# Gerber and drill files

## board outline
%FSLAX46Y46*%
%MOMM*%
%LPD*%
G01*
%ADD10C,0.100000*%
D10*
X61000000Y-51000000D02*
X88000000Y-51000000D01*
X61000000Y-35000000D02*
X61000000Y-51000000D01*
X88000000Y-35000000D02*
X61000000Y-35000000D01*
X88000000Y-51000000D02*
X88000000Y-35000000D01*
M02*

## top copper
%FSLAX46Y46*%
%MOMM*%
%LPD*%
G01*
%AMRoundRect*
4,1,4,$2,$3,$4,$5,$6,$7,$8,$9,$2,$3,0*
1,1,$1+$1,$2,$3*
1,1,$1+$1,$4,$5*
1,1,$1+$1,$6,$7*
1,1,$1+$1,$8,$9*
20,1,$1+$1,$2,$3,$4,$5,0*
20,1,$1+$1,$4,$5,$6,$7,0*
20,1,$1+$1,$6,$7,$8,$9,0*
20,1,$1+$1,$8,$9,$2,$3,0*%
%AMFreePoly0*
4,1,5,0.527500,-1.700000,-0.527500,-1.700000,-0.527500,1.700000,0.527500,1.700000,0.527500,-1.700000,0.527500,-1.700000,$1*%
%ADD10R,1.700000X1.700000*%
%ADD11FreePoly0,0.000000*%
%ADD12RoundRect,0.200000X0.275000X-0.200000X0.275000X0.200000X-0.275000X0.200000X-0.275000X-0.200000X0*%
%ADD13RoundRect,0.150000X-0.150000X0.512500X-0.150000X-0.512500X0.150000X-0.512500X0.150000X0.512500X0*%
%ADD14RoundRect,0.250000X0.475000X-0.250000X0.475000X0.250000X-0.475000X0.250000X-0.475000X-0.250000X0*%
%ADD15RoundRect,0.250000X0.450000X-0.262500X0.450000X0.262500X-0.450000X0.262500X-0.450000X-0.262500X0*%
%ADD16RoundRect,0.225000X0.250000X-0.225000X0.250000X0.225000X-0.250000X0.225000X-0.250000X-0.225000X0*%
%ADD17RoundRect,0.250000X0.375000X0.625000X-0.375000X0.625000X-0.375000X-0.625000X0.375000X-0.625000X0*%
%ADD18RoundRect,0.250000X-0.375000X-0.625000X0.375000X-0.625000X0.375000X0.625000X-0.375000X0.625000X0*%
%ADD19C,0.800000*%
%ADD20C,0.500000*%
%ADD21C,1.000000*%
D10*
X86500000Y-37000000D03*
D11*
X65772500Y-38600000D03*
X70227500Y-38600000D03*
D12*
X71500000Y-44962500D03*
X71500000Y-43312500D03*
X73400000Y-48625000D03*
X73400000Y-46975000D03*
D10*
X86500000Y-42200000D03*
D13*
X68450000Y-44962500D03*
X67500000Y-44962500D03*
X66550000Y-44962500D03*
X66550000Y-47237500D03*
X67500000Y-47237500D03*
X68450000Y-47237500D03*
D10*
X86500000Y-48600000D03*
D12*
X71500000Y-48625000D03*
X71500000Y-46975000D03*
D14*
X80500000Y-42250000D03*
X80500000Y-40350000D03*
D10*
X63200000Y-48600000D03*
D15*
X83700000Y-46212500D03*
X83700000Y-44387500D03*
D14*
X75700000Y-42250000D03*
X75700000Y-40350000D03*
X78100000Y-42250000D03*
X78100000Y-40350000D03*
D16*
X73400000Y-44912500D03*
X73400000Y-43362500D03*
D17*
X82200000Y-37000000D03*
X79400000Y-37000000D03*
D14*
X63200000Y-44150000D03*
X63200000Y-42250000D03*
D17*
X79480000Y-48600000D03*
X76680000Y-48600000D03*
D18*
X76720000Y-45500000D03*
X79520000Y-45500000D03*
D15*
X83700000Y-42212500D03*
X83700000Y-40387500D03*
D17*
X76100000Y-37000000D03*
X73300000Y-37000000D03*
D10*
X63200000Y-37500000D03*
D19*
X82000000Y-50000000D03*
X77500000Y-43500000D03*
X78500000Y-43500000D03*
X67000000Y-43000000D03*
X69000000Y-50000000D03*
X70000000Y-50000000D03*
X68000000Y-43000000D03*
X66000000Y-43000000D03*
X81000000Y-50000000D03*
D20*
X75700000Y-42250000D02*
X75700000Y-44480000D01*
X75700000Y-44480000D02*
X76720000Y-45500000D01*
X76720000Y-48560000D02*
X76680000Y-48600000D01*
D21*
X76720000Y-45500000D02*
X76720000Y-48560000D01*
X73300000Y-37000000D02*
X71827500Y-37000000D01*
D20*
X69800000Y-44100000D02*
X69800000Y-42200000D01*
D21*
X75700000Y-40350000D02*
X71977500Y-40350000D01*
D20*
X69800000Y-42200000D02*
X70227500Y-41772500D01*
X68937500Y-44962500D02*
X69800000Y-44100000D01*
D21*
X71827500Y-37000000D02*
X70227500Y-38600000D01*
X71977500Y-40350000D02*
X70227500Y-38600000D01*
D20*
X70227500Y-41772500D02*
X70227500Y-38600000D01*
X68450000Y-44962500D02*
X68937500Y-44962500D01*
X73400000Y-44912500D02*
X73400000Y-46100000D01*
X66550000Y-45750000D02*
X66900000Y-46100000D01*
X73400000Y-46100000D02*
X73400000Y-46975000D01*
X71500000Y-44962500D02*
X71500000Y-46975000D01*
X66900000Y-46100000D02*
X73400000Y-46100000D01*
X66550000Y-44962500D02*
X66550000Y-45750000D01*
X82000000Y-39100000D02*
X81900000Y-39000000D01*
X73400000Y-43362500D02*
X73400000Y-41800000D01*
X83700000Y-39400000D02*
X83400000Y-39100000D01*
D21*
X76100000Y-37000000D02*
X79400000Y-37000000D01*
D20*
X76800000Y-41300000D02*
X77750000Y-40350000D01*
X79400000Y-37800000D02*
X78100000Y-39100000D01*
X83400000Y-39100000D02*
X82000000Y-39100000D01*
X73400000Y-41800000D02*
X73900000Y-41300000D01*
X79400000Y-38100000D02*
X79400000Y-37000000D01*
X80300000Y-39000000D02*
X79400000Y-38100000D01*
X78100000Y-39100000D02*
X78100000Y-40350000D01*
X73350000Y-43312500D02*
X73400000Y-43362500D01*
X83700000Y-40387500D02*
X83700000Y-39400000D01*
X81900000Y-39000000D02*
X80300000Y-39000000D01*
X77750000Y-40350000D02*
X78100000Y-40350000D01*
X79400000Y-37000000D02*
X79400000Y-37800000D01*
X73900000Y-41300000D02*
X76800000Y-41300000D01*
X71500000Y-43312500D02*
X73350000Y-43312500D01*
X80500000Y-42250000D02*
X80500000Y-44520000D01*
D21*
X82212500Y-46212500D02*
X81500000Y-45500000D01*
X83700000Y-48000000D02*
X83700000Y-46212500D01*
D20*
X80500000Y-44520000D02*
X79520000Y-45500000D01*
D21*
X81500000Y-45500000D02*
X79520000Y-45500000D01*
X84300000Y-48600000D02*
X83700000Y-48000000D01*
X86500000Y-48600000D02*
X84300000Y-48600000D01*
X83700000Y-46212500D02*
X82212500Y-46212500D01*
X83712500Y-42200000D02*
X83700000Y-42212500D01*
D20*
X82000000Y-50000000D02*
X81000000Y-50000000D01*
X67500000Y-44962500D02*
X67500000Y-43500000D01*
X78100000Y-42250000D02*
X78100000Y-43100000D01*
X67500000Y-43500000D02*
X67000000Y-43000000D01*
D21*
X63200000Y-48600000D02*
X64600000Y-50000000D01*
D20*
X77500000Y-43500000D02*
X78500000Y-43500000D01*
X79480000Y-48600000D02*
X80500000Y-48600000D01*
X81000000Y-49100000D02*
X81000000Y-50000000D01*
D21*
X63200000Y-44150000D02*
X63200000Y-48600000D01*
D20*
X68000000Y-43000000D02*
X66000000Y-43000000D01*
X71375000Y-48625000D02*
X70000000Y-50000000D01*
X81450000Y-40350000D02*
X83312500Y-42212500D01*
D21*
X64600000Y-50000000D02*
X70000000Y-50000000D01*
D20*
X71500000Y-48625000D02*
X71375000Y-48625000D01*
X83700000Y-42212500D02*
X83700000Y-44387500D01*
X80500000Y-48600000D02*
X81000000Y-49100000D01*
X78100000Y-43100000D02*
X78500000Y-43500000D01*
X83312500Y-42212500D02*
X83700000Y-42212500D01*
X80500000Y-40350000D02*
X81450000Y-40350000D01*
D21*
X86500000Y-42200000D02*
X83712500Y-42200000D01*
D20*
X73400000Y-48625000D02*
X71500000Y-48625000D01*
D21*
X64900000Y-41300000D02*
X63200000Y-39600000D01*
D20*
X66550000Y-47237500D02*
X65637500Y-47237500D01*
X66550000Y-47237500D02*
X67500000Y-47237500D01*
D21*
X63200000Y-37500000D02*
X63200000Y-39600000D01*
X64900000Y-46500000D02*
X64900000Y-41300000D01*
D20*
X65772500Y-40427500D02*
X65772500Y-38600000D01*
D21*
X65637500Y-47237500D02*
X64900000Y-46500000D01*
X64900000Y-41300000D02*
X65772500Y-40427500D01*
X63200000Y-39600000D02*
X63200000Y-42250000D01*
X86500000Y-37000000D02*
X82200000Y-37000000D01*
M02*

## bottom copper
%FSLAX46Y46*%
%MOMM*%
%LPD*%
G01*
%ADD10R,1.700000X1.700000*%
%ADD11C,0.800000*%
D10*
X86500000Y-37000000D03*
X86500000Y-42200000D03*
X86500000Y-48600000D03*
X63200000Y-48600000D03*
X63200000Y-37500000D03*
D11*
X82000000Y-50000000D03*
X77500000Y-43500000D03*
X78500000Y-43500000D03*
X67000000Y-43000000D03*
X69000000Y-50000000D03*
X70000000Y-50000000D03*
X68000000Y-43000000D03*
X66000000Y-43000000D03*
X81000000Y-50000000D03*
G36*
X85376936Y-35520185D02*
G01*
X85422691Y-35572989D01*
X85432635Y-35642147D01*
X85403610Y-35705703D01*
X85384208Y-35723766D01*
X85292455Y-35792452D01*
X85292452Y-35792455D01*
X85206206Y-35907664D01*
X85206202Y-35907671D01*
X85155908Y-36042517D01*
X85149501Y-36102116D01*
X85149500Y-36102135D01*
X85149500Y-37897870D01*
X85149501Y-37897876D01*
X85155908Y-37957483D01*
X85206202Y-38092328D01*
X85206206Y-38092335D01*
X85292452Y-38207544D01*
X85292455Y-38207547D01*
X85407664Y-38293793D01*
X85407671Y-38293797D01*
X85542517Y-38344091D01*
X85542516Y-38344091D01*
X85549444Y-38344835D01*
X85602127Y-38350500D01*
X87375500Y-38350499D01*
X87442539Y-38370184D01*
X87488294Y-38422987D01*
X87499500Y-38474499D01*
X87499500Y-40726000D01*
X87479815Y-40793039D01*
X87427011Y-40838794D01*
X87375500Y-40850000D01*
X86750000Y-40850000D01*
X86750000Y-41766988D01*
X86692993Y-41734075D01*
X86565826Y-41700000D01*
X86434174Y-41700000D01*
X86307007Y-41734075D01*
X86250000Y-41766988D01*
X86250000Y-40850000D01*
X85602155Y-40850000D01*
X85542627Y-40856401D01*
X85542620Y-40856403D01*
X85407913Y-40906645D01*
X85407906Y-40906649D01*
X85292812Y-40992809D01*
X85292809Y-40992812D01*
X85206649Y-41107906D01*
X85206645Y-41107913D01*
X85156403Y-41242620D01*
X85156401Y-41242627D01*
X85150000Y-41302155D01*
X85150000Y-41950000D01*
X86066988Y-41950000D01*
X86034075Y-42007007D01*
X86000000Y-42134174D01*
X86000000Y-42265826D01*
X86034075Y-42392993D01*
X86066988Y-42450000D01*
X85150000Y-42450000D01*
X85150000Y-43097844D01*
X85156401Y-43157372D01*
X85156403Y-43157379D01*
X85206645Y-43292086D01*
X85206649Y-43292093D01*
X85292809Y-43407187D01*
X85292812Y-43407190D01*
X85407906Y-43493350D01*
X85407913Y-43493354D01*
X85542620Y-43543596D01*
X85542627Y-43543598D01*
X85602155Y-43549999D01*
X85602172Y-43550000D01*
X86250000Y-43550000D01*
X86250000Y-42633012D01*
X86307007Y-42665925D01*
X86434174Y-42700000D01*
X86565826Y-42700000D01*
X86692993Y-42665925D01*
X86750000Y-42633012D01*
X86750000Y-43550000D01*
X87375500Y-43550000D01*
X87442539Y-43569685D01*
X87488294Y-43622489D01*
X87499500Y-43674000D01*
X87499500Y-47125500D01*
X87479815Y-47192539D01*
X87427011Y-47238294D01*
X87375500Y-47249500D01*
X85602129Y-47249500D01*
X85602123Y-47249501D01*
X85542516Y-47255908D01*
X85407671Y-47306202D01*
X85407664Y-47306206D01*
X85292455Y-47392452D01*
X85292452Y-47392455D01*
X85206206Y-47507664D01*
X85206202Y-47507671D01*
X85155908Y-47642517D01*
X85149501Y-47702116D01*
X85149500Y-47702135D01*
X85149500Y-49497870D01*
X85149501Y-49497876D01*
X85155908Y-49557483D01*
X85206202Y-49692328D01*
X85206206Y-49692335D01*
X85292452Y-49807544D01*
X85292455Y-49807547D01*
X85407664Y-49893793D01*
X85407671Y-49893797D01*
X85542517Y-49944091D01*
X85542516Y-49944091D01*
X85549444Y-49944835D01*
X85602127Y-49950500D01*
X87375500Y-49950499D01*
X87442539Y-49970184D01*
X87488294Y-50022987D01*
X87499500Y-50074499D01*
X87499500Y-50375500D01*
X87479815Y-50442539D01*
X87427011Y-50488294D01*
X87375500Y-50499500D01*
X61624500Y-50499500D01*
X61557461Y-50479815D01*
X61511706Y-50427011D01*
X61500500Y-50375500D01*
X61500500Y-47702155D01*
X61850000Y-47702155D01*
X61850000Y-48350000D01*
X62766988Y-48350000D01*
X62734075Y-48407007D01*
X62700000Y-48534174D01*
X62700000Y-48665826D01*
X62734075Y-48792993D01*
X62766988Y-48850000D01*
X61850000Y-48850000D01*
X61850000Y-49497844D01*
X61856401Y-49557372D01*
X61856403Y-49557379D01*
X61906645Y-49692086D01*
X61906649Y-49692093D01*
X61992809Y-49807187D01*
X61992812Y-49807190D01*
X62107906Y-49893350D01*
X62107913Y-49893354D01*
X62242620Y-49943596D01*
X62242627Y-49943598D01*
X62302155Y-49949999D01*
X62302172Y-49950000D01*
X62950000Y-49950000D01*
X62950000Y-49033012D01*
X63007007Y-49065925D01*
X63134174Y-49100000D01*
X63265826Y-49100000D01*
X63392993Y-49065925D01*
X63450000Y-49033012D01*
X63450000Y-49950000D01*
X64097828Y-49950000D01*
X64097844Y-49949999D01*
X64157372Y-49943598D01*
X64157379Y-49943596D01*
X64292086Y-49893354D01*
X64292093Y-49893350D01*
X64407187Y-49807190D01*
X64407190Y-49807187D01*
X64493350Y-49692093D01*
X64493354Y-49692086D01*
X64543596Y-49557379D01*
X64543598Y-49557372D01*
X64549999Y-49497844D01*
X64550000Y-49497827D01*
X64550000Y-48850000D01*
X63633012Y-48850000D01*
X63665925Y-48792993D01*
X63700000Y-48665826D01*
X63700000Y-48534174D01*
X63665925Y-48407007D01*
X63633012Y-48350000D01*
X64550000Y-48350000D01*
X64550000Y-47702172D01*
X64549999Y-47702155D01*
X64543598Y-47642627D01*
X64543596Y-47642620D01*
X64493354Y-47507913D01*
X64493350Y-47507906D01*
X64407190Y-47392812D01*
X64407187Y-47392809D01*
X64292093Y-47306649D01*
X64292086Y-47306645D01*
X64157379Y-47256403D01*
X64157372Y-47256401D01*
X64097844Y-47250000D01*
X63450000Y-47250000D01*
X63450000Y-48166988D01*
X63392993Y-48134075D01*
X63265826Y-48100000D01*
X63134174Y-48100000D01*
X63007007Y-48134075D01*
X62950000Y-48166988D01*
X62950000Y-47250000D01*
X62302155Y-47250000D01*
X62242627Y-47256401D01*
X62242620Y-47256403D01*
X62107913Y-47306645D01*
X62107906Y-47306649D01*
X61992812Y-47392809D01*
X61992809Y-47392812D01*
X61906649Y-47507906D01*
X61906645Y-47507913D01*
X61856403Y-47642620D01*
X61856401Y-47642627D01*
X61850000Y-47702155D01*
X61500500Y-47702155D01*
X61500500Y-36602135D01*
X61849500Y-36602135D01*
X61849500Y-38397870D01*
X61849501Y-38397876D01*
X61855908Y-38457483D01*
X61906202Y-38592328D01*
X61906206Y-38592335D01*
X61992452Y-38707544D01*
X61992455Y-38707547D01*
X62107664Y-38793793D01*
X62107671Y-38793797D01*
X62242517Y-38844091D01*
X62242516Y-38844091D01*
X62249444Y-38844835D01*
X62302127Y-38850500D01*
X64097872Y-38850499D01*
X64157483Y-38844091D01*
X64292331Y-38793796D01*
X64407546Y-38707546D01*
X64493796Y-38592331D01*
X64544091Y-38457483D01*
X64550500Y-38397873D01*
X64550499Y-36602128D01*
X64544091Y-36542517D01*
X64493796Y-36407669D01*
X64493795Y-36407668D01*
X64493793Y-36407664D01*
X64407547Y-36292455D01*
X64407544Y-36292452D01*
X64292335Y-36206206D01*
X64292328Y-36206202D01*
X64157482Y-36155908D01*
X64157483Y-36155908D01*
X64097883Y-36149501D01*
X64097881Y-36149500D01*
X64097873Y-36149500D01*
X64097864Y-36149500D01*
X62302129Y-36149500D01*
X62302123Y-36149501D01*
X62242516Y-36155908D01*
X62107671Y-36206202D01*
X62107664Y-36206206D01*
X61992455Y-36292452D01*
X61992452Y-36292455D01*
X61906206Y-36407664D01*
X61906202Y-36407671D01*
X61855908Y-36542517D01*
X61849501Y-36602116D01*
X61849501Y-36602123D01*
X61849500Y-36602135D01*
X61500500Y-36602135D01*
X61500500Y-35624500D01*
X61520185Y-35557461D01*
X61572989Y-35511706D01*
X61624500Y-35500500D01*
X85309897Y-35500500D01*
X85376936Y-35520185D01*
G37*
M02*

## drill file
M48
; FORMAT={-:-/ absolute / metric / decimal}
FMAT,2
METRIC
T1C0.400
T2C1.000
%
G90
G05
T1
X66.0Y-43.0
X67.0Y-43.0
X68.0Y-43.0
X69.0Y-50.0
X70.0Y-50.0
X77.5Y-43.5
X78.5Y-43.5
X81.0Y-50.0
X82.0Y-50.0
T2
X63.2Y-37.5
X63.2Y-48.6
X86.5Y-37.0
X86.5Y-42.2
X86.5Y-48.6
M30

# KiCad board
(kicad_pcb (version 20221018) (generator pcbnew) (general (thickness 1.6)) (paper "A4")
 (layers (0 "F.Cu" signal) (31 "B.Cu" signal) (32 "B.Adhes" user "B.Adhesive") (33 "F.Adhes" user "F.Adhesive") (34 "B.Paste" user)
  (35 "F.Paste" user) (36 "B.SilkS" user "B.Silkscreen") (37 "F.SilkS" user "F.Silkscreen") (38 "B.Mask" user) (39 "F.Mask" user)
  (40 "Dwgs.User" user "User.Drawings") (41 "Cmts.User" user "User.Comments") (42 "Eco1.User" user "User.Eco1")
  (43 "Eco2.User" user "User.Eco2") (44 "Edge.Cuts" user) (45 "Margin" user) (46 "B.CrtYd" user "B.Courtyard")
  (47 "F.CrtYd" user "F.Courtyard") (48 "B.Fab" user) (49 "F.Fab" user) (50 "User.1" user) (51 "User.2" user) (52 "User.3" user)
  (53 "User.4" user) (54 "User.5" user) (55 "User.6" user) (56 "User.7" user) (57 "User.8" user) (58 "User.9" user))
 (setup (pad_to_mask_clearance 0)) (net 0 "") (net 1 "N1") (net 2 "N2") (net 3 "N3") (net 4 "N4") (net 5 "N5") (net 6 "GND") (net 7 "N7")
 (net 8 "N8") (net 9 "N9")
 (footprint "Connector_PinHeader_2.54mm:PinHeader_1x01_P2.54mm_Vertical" (layer "F.Cu") (at 86.5 37)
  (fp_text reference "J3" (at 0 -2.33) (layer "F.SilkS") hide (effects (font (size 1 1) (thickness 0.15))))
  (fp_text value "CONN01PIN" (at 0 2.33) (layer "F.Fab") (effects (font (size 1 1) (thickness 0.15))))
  (pad "1" thru_hole rect (at 0 0) (size 1.7 1.7) (drill 1) (layers "*.Cu" "*.Mask") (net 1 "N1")))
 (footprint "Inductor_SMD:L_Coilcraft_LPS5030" (layer "F.Cu") (at 68 38.6)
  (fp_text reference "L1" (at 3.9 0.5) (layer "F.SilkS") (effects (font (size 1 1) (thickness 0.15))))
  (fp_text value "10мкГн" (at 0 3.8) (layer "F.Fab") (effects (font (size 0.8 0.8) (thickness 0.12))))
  (pad "1" smd custom (at -2.2275 0) (size 1.055 3.4) (layers "F.Cu" "F.Paste" "F.Mask") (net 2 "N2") (zone_connect 2)
   (options (clearance outline) (anchor rect)) (primitives))
  (pad "2" smd custom (at 2.2275 0) (size 1.055 3.4) (layers "F.Cu" "F.Paste" "F.Mask") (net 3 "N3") (zone_connect 2)
   (options (clearance outline) (anchor rect)) (primitives)))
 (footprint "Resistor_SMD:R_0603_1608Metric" (layer "F.Cu") (at 71.5 44.1375 90)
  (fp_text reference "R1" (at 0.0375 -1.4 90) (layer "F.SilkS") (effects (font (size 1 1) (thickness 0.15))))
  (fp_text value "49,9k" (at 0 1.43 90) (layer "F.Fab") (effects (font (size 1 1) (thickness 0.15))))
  (pad "1" smd roundrect (at -0.825 0 90) (size 0.8 0.95) (layers "F.Cu" "F.Paste" "F.Mask") (roundrect_rratio 0.25) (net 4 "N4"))
  (pad "2" smd roundrect (at 0.825 0 90) (size 0.8 0.95) (layers "F.Cu" "F.Paste" "F.Mask") (roundrect_rratio 0.25) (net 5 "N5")))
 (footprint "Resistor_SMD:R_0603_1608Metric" (layer "F.Cu") (at 73.4 47.8 90)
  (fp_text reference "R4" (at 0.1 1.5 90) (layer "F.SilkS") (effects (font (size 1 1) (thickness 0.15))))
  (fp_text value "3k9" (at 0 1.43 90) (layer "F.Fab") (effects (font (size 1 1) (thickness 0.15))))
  (pad "1" smd roundrect (at -0.825 0 90) (size 0.8 0.95) (layers "F.Cu" "F.Paste" "F.Mask") (roundrect_rratio 0.25) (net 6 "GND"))
  (pad "2" smd roundrect (at 0.825 0 90) (size 0.8 0.95) (layers "F.Cu" "F.Paste" "F.Mask") (roundrect_rratio 0.25) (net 4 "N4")))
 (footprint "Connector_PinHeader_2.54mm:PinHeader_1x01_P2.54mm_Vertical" (layer "F.Cu") (at 86.5 42.2)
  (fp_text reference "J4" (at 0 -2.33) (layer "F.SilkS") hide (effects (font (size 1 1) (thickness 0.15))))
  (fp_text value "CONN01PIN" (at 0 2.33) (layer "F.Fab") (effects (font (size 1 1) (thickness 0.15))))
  (pad "1" thru_hole rect (at 0 0) (size 1.7 1.7) (drill 1) (layers "*.Cu" "*.Mask") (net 6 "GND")))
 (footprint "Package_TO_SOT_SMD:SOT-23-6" (layer "F.Cu") (at 67.5 46.1 -90)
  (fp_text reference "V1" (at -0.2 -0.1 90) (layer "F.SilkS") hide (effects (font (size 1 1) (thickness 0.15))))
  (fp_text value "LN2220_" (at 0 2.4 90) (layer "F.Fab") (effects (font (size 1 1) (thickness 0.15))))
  (pad "1" smd roundrect (at -1.1375 -0.95 270) (size 1.325 0.6) (layers "F.Cu" "F.Paste" "F.Mask") (roundrect_rratio 0.25) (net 3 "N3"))
  (pad "2" smd roundrect (at -1.1375 0 270) (size 1.325 0.6) (layers "F.Cu" "F.Paste" "F.Mask") (roundrect_rratio 0.25) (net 6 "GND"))
  (pad "3" smd roundrect (at -1.1375 0.95 270) (size 1.325 0.6) (layers "F.Cu" "F.Paste" "F.Mask") (roundrect_rratio 0.25) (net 4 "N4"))
  (pad "4" smd roundrect (at 1.1375 0.95 270) (size 1.325 0.6) (layers "F.Cu" "F.Paste" "F.Mask") (roundrect_rratio 0.25) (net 2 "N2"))
  (pad "5" smd roundrect (at 1.1375 0 270) (size 1.325 0.6) (layers "F.Cu" "F.Paste" "F.Mask") (roundrect_rratio 0.25) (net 2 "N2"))
  (pad "6" smd roundrect (at 1.1375 -0.95 270) (size 1.325 0.6) (layers "F.Cu" "F.Paste" "F.Mask") (roundrect_rratio 0.25) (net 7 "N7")))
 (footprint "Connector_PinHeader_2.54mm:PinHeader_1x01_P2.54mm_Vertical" (layer "F.Cu") (at 86.5 48.6)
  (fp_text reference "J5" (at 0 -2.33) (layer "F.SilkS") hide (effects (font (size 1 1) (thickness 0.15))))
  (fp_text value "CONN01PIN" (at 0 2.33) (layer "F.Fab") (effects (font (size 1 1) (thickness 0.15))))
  (pad "1" thru_hole rect (at 0 0) (size 1.7 1.7) (drill 1) (layers "*.Cu" "*.Mask") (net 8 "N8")))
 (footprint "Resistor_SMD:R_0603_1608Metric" (layer "F.Cu") (at 71.5 47.8 90)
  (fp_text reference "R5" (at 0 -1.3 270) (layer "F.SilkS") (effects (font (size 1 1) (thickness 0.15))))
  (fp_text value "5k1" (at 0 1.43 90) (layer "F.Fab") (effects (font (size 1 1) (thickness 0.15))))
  (pad "1" smd roundrect (at -0.825 0 90) (size 0.8 0.95) (layers "F.Cu" "F.Paste" "F.Mask") (roundrect_rratio 0.25) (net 6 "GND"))
  (pad "2" smd roundrect (at 0.825 0 90) (size 0.8 0.95) (layers "F.Cu" "F.Paste" "F.Mask") (roundrect_rratio 0.25) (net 4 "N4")))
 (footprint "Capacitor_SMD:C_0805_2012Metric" (layer "F.Cu") (at 80.5 41.3 90)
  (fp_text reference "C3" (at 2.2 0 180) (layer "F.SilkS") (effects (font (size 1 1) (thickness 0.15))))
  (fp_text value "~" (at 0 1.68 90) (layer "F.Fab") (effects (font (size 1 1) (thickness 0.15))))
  (pad "1" smd roundrect (at -0.95 0 90) (size 1 1.45) (layers "F.Cu" "F.Paste" "F.Mask") (roundrect_rratio 0.25) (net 8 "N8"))
  (pad "2" smd roundrect (at 0.95 0 90) (size 1 1.45) (layers "F.Cu" "F.Paste" "F.Mask") (roundrect_rratio 0.25) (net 6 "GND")))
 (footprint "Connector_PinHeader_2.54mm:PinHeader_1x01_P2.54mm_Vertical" (layer "F.Cu") (at 63.2 48.6)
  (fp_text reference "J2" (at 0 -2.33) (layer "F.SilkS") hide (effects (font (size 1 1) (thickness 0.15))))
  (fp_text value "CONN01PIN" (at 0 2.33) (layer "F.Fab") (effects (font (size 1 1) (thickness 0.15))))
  (pad "1" thru_hole rect (at 0 0) (size 1.7 1.7) (drill 1) (layers "*.Cu" "*.Mask") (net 6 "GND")))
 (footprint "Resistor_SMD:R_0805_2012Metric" (layer "F.Cu") (at 83.7 45.3 90)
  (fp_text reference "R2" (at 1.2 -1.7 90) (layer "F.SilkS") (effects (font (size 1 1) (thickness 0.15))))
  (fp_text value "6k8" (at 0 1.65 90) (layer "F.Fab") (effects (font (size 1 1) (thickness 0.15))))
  (pad "1" smd roundrect (at -0.9125 0 90) (size 1.025 1.4) (layers "F.Cu" "F.Paste" "F.Mask") (roundrect_rratio 0.243902) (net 8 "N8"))
  (pad "2" smd roundrect (at 0.9125 0 90) (size 1.025 1.4) (layers "F.Cu" "F.Paste" "F.Mask") (roundrect_rratio 0.243902) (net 6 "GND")))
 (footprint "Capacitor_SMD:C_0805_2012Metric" (layer "F.Cu") (at 75.7 41.3 90)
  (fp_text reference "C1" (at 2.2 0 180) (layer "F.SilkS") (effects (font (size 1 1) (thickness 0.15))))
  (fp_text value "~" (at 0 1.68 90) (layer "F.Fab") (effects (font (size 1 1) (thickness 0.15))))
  (pad "1" smd roundrect (at -0.95 0 90) (size 1 1.45) (layers "F.Cu" "F.Paste" "F.Mask") (roundrect_rratio 0.25) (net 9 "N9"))
  (pad "2" smd roundrect (at 0.95 0 90) (size 1 1.45) (layers "F.Cu" "F.Paste" "F.Mask") (roundrect_rratio 0.25) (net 3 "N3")))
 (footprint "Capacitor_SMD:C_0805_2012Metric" (layer "F.Cu") (at 78.1 41.3 90)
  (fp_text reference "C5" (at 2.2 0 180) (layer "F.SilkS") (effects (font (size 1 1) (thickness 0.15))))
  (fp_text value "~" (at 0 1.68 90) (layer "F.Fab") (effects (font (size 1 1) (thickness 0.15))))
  (pad "1" smd roundrect (at -0.95 0 90) (size 1 1.45) (layers "F.Cu" "F.Paste" "F.Mask") (roundrect_rratio 0.25) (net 6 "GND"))
  (pad "2" smd roundrect (at 0.95 0 90) (size 1 1.45) (layers "F.Cu" "F.Paste" "F.Mask") (roundrect_rratio 0.25) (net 5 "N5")))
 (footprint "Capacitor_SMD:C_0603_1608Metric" (layer "F.Cu") (at 73.4 44.1375 90)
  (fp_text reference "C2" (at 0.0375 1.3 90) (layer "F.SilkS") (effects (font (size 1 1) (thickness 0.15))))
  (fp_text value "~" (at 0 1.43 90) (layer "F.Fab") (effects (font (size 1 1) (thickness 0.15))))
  (pad "1" smd roundrect (at -0.775 0 90) (size 0.9 0.95) (layers "F.Cu" "F.Paste" "F.Mask") (roundrect_rratio 0.25) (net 4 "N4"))
  (pad "2" smd roundrect (at 0.775 0 90) (size 0.9 0.95) (layers "F.Cu" "F.Paste" "F.Mask") (roundrect_rratio 0.25) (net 5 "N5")))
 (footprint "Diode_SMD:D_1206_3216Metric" (layer "F.Cu") (at 80.8 37 180)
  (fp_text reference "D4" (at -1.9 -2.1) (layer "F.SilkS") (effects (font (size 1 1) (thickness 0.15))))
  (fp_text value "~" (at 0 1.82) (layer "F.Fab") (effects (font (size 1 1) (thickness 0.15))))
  (pad "1" smd roundrect (at -1.4 0 180) (size 1.25 1.75) (layers "F.Cu" "F.Paste" "F.Mask") (roundrect_rratio 0.2) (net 1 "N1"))
  (pad "2" smd roundrect (at 1.4 0 180) (size 1.25 1.75) (layers "F.Cu" "F.Paste" "F.Mask") (roundrect_rratio 0.2) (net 5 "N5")))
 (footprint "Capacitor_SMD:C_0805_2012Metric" (layer "F.Cu") (at 63.2 43.2 90)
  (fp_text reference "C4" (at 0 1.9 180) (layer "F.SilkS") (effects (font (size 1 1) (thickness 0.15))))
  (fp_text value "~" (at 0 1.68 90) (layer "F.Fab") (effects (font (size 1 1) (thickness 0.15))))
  (pad "1" smd roundrect (at -0.95 0 90) (size 1 1.45) (layers "F.Cu" "F.Paste" "F.Mask") (roundrect_rratio 0.25) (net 6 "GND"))
  (pad "2" smd roundrect (at 0.95 0 90) (size 1 1.45) (layers "F.Cu" "F.Paste" "F.Mask") (roundrect_rratio 0.25) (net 2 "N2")))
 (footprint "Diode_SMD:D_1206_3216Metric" (layer "F.Cu") (at 78.08 48.6 180)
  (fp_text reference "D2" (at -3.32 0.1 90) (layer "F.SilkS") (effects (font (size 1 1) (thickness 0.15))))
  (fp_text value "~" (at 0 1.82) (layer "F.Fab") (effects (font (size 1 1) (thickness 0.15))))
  (pad "1" smd roundrect (at -1.4 0 180) (size 1.25 1.75) (layers "F.Cu" "F.Paste" "F.Mask") (roundrect_rratio 0.2) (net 6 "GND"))
  (pad "2" smd roundrect (at 1.4 0 180) (size 1.25 1.75) (layers "F.Cu" "F.Paste" "F.Mask") (roundrect_rratio 0.2) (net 9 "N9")))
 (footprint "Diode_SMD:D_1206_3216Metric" (layer "F.Cu") (at 78.12 45.5)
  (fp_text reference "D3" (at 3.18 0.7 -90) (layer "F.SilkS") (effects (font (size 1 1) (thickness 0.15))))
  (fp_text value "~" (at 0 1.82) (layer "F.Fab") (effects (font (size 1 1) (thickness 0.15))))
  (pad "1" smd roundrect (at -1.4 0) (size 1.25 1.75) (layers "F.Cu" "F.Paste" "F.Mask") (roundrect_rratio 0.2) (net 9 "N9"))
  (pad "2" smd roundrect (at 1.4 0) (size 1.25 1.75) (layers "F.Cu" "F.Paste" "F.Mask") (roundrect_rratio 0.2) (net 8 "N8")))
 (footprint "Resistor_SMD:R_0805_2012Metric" (layer "F.Cu") (at 83.7 41.3 90)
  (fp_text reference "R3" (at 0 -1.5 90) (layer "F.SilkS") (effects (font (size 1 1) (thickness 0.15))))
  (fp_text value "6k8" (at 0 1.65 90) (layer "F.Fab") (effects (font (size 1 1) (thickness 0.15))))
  (pad "1" smd roundrect (at -0.9125 0 90) (size 1.025 1.4) (layers "F.Cu" "F.Paste" "F.Mask") (roundrect_rratio 0.243902) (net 6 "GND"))
  (pad "2" smd roundrect (at 0.9125 0 90) (size 1.025 1.4) (layers "F.Cu" "F.Paste" "F.Mask") (roundrect_rratio 0.243902) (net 5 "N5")))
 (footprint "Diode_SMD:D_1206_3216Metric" (layer "F.Cu") (at 74.7 37 180)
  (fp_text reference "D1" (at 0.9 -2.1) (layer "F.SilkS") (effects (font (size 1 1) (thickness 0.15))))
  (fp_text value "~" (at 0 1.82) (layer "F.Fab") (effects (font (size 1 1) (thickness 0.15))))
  (pad "1" smd roundrect (at -1.4 0 180) (size 1.25 1.75) (layers "F.Cu" "F.Paste" "F.Mask") (roundrect_rratio 0.2) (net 5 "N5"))
  (pad "2" smd roundrect (at 1.4 0 180) (size 1.25 1.75) (layers "F.Cu" "F.Paste" "F.Mask") (roundrect_rratio 0.2) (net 3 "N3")))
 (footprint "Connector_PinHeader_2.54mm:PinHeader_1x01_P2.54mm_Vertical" (layer "F.Cu") (at 63.2 37.5)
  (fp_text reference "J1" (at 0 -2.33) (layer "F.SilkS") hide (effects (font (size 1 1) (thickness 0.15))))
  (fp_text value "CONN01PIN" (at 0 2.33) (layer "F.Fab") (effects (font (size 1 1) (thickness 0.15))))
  (pad "1" thru_hole rect (at 0 0) (size 1.7 1.7) (drill 1) (layers "*.Cu" "*.Mask") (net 2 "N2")))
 (gr_line (start 61 51) (end 88 51) (stroke (width 0.1) (type default)) (layer "Edge.Cuts"))
 (gr_line (start 61 35) (end 61 51) (stroke (width 0.1) (type default)) (layer "Edge.Cuts"))
 (gr_line (start 88 35) (end 61 35) (stroke (width 0.1) (type default)) (layer "Edge.Cuts"))
 (gr_line (start 88 51) (end 88 35) (stroke (width 0.1) (type default)) (layer "Edge.Cuts"))
 (segment (start 75.7 42.25) (end 75.7 44.48) (width 0.5) (layer "F.Cu") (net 9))
 (segment (start 75.7 44.48) (end 76.72 45.5) (width 0.5) (layer "F.Cu") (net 9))
 (segment (start 76.72 48.56) (end 76.68 48.6) (width 0.5) (layer "F.Cu") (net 9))
 (segment (start 76.72 45.5) (end 76.72 48.56) (width 1) (layer "F.Cu") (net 9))
 (segment (start 73.3 37) (end 71.8275 37) (width 1) (layer "F.Cu") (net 3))
 (segment (start 69.8 44.1) (end 69.8 42.2) (width 0.5) (layer "F.Cu") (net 3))
 (segment (start 75.7 40.35) (end 71.9775 40.35) (width 1) (layer "F.Cu") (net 3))
 (segment (start 69.8 42.2) (end 70.2275 41.7725) (width 0.5) (layer "F.Cu") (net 3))
 (segment (start 68.9375 44.9625) (end 69.8 44.1) (width 0.5) (layer "F.Cu") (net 3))
 (segment (start 71.8275 37) (end 70.2275 38.6) (width 1) (layer "F.Cu") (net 3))
 (segment (start 71.9775 40.35) (end 70.2275 38.6) (width 1) (layer "F.Cu") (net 3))
 (segment (start 70.2275 41.7725) (end 70.2275 38.6) (width 0.5) (layer "F.Cu") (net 3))
 (segment (start 68.45 44.9625) (end 68.9375 44.9625) (width 0.5) (layer "F.Cu") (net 3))
 (segment (start 73.4 44.9125) (end 73.4 46.1) (width 0.5) (layer "F.Cu") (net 4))
 (segment (start 66.55 45.75) (end 66.9 46.1) (width 0.5) (layer "F.Cu") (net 4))
 (segment (start 73.4 46.1) (end 73.4 46.975) (width 0.5) (layer "F.Cu") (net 4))
 (segment (start 71.5 44.9625) (end 71.5 46.975) (width 0.5) (layer "F.Cu") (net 4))
 (segment (start 66.9 46.1) (end 73.4 46.1) (width 0.5) (layer "F.Cu") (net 4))
 (segment (start 66.55 44.9625) (end 66.55 45.75) (width 0.5) (layer "F.Cu") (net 4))
 (segment (start 82 39.1) (end 81.9 39) (width 0.5) (layer "F.Cu") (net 5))
 (segment (start 73.4 43.3625) (end 73.4 41.8) (width 0.5) (layer "F.Cu") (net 5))
 (segment (start 83.7 39.4) (end 83.4 39.1) (width 0.5) (layer "F.Cu") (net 5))
 (segment (start 76.1 37) (end 79.4 37) (width 1) (layer "F.Cu") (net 5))
 (segment (start 76.8 41.3) (end 77.75 40.35) (width 0.5) (layer "F.Cu") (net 5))
 (segment (start 79.4 37.8) (end 78.1 39.1) (width 0.5) (layer "F.Cu") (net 5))
 (segment (start 83.4 39.1) (end 82 39.1) (width 0.5) (layer "F.Cu") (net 5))
 (segment (start 73.4 41.8) (end 73.9 41.3) (width 0.5) (layer "F.Cu") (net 5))
 (segment (start 79.4 38.1) (end 79.4 37) (width 0.5) (layer "F.Cu") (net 5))
 (segment (start 80.3 39) (end 79.4 38.1) (width 0.5) (layer "F.Cu") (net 5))
 (segment (start 78.1 39.1) (end 78.1 40.35) (width 0.5) (layer "F.Cu") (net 5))
 (segment (start 73.35 43.3125) (end 73.4 43.3625) (width 0.5) (layer "F.Cu") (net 5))
 (segment (start 83.7 40.3875) (end 83.7 39.4) (width 0.5) (layer "F.Cu") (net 5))
 (segment (start 81.9 39) (end 80.3 39) (width 0.5) (layer "F.Cu") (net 5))
 (segment (start 77.75 40.35) (end 78.1 40.35) (width 0.5) (layer "F.Cu") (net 5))
 (segment (start 79.4 37) (end 79.4 37.8) (width 0.5) (layer "F.Cu") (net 5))
 (segment (start 73.9 41.3) (end 76.8 41.3) (width 0.5) (layer "F.Cu") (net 5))
 (segment (start 71.5 43.3125) (end 73.35 43.3125) (width 0.5) (layer "F.Cu") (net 5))
 (segment (start 80.5 42.25) (end 80.5 44.52) (width 0.5) (layer "F.Cu") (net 8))
 (segment (start 82.2125 46.2125) (end 81.5 45.5) (width 1) (layer "F.Cu") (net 8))
 (segment (start 83.7 48) (end 83.7 46.2125) (width 1) (layer "F.Cu") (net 8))
 (segment (start 80.5 44.52) (end 79.52 45.5) (width 0.5) (layer "F.Cu") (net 8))
 (segment (start 81.5 45.5) (end 79.52 45.5) (width 1) (layer "F.Cu") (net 8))
 (segment (start 84.3 48.6) (end 83.7 48) (width 1) (layer "F.Cu") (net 8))
 (segment (start 86.5 48.6) (end 84.3 48.6) (width 1) (layer "F.Cu") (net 8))
 (segment (start 83.7 46.2125) (end 82.2125 46.2125) (width 1) (layer "F.Cu") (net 8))
 (segment (start 83.7125 42.2) (end 83.7 42.2125) (width 1) (layer "F.Cu") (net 6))
 (segment (start 82 50) (end 81 50) (width 0.5) (layer "F.Cu") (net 6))
 (segment (start 67.5 44.9625) (end 67.5 43.5) (width 0.5) (layer "F.Cu") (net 6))
 (segment (start 78.1 42.25) (end 78.1 43.1) (width 0.5) (layer "F.Cu") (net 6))
 (segment (start 67.5 43.5) (end 67 43) (width 0.5) (layer "F.Cu") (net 6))
 (segment (start 63.2 48.6) (end 64.6 50) (width 1) (layer "F.Cu") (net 6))
 (segment (start 77.5 43.5) (end 78.5 43.5) (width 0.5) (layer "F.Cu") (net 6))
 (segment (start 79.48 48.6) (end 80.5 48.6) (width 0.5) (layer "F.Cu") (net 6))
 (segment (start 81 49.1) (end 81 50) (width 0.5) (layer "F.Cu") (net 6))
 (segment (start 63.2 44.15) (end 63.2 48.6) (width 1) (layer "F.Cu") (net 6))
 (segment (start 68 43) (end 66 43) (width 0.5) (layer "F.Cu") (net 6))
 (segment (start 71.375 48.625) (end 70 50) (width 0.5) (layer "F.Cu") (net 6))
 (segment (start 81.45 40.35) (end 83.3125 42.2125) (width 0.5) (layer "F.Cu") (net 6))
 (segment (start 64.6 50) (end 70 50) (width 1) (layer "F.Cu") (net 6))
 (segment (start 71.5 48.625) (end 71.375 48.625) (width 0.5) (layer "F.Cu") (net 6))
 (segment (start 83.7 42.2125) (end 83.7 44.3875) (width 0.5) (layer "F.Cu") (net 6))
 (segment (start 80.5 48.6) (end 81 49.1) (width 0.5) (layer "F.Cu") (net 6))
 (segment (start 78.1 43.1) (end 78.5 43.5) (width 0.5) (layer "F.Cu") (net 6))
 (segment (start 83.3125 42.2125) (end 83.7 42.2125) (width 0.5) (layer "F.Cu") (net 6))
 (segment (start 80.5 40.35) (end 81.45 40.35) (width 0.5) (layer "F.Cu") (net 6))
 (segment (start 86.5 42.2) (end 83.7125 42.2) (width 1) (layer "F.Cu") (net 6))
 (segment (start 73.4 48.625) (end 71.5 48.625) (width 0.5) (layer "F.Cu") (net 6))
 (via (at 82 50) (size 0.8) (drill 0.4) (layers "F.Cu" "B.Cu") (free) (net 6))
 (via (at 77.5 43.5) (size 0.8) (drill 0.4) (layers "F.Cu" "B.Cu") (free) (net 6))
 (via (at 78.5 43.5) (size 0.8) (drill 0.4) (layers "F.Cu" "B.Cu") (free) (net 6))
 (via (at 67 43) (size 0.8) (drill 0.4) (layers "F.Cu" "B.Cu") (free) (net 6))
 (via (at 69 50) (size 0.8) (drill 0.4) (layers "F.Cu" "B.Cu") (free) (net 6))
 (via (at 70 50) (size 0.8) (drill 0.4) (layers "F.Cu" "B.Cu") (free) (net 6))
 (via (at 68 43) (size 0.8) (drill 0.4) (layers "F.Cu" "B.Cu") (free) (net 6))
 (via (at 66 43) (size 0.8) (drill 0.4) (layers "F.Cu" "B.Cu") (free) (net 6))
 (via (at 81 50) (size 0.8) (drill 0.4) (layers "F.Cu" "B.Cu") (free) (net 6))
 (segment (start 64.9 41.3) (end 63.2 39.6) (width 1) (layer "F.Cu") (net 2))
 (segment (start 66.55 47.2375) (end 65.6375 47.2375) (width 0.5) (layer "F.Cu") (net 2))
 (segment (start 66.55 47.2375) (end 67.5 47.2375) (width 0.5) (layer "F.Cu") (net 2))
 (segment (start 63.2 37.5) (end 63.2 39.6) (width 1) (layer "F.Cu") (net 2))
 (segment (start 64.9 46.5) (end 64.9 41.3) (width 1) (layer "F.Cu") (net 2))
 (segment (start 65.7725 40.4275) (end 65.7725 38.6) (width 0.5) (layer "F.Cu") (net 2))
 (segment (start 65.6375 47.2375) (end 64.9 46.5) (width 1) (layer "F.Cu") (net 2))
 (segment (start 64.9 41.3) (end 65.7725 40.4275) (width 1) (layer "F.Cu") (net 2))
 (segment (start 63.2 39.6) (end 63.2 42.25) (width 1) (layer "F.Cu") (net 2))
 (segment (start 86.5 37) (end 82.2 37) (width 1) (layer "F.Cu") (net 1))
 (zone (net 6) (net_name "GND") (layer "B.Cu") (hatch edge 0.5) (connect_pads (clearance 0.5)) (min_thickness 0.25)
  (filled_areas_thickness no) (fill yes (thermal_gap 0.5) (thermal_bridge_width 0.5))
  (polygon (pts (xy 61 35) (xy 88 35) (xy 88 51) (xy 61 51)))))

